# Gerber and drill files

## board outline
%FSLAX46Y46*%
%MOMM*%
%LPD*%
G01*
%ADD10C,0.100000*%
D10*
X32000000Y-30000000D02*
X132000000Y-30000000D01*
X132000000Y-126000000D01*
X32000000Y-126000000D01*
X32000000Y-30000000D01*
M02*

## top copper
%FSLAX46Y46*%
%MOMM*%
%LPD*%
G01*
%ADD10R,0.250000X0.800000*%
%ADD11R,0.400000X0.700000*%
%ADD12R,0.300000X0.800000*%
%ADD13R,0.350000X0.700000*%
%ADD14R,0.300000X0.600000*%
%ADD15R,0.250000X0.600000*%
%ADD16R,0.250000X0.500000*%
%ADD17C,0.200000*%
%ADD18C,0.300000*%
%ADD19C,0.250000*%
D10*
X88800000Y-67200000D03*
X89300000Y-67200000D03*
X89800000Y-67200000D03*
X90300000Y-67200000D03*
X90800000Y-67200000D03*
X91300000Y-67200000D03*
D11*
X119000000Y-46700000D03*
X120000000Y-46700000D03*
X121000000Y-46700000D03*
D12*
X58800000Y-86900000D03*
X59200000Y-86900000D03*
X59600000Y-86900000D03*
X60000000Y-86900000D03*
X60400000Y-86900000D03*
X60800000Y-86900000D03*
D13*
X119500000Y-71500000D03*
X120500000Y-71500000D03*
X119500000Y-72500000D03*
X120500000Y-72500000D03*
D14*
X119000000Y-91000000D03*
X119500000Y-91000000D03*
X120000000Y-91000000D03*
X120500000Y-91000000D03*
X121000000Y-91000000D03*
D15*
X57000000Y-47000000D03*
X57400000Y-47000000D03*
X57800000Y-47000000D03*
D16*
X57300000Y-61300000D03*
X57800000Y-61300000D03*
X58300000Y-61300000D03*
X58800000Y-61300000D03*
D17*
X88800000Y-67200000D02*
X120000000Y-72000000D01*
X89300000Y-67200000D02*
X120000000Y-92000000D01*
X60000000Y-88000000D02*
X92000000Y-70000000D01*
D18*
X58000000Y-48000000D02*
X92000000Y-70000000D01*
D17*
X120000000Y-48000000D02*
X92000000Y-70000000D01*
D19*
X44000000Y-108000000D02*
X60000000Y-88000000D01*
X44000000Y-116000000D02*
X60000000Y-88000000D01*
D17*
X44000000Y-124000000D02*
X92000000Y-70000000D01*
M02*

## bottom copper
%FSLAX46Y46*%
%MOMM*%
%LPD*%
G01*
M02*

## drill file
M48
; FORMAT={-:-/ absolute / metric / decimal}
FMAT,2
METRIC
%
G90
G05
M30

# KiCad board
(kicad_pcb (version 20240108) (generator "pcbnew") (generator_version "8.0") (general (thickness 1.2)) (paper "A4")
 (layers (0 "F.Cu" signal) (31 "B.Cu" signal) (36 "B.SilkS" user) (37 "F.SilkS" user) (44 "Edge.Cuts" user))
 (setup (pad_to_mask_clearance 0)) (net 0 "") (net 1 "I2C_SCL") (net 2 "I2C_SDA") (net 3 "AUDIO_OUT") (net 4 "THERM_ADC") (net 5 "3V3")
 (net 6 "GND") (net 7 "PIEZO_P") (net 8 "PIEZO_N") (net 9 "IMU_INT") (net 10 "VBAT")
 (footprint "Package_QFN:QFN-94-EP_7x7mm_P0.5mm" (layer "F.Cu") (at 92 70)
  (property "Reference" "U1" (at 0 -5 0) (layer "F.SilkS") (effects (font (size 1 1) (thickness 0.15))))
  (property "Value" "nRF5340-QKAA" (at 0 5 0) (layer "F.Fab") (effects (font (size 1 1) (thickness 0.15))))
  (pad "1" smd rect (at -3.2 -2.8) (size 0.25 0.8) (layers "F.Cu" "F.Paste" "F.Mask") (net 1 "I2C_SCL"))
  (pad "2" smd rect (at -2.7 -2.8) (size 0.25 0.8) (layers "F.Cu" "F.Paste" "F.Mask") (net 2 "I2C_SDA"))
  (pad "3" smd rect (at -2.2 -2.8) (size 0.25 0.8) (layers "F.Cu" "F.Paste" "F.Mask") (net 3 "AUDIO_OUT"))
  (pad "4" smd rect (at -1.7 -2.8) (size 0.25 0.8) (layers "F.Cu" "F.Paste" "F.Mask") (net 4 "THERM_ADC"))
  (pad "5" smd rect (at -1.2 -2.8) (size 0.25 0.8) (layers "F.Cu" "F.Paste" "F.Mask") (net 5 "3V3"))
  (pad "6" smd rect (at -0.7 -2.8) (size 0.25 0.8) (layers "F.Cu" "F.Paste" "F.Mask") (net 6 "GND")))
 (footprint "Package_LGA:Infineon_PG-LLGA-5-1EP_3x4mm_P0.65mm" (layer "F.Cu") (at 120 48)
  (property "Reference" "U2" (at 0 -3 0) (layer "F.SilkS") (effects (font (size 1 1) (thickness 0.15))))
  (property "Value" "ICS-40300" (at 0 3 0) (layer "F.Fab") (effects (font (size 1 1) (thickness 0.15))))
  (pad "1" smd rect (at -1.0 -1.3) (size 0.4 0.7) (layers "F.Cu" "F.Paste" "F.Mask") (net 3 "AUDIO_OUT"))
  (pad "2" smd rect (at 0.0 -1.3) (size 0.4 0.7) (layers "F.Cu" "F.Paste" "F.Mask") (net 5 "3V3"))
  (pad "3" smd rect (at 1.0 -1.3) (size 0.4 0.7) (layers "F.Cu" "F.Paste" "F.Mask") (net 6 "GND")))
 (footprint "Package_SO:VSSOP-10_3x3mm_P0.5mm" (layer "F.Cu") (at 60 88)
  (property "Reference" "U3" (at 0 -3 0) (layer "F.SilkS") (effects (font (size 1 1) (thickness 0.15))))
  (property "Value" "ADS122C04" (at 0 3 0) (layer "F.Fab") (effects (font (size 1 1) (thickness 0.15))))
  (pad "1" smd rect (at -1.2 -1.1) (size 0.3 0.8) (layers "F.Cu" "F.Paste" "F.Mask") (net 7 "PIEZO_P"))
  (pad "2" smd rect (at -0.8 -1.1) (size 0.3 0.8) (layers "F.Cu" "F.Paste" "F.Mask") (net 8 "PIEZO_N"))
  (pad "3" smd rect (at -0.4 -1.1) (size 0.3 0.8) (layers "F.Cu" "F.Paste" "F.Mask") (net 1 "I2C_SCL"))
  (pad "4" smd rect (at 0.0 -1.1) (size 0.3 0.8) (layers "F.Cu" "F.Paste" "F.Mask") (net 2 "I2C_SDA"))
  (pad "5" smd rect (at 0.4 -1.1) (size 0.3 0.8) (layers "F.Cu" "F.Paste" "F.Mask") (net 5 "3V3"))
  (pad "6" smd rect (at 0.8 -1.1) (size 0.3 0.8) (layers "F.Cu" "F.Paste" "F.Mask") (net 6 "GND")))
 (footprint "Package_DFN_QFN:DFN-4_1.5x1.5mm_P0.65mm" (layer "F.Cu") (at 120 72)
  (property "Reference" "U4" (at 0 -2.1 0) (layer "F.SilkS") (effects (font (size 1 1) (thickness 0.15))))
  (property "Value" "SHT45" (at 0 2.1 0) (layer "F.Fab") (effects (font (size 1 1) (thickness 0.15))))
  (pad "1" smd rect (at -0.5 -0.5) (size 0.35 0.7) (layers "F.Cu" "F.Paste" "F.Mask") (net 1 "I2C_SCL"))
  (pad "2" smd rect (at 0.5 -0.5) (size 0.35 0.7) (layers "F.Cu" "F.Paste" "F.Mask") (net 2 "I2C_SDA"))
  (pad "3" smd rect (at -0.5 0.5) (size 0.35 0.7) (layers "F.Cu" "F.Paste" "F.Mask") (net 5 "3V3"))
  (pad "4" smd rect (at 0.5 0.5) (size 0.35 0.7) (layers "F.Cu" "F.Paste" "F.Mask") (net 6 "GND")))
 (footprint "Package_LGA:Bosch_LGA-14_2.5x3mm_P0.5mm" (layer "F.Cu") (at 120 92)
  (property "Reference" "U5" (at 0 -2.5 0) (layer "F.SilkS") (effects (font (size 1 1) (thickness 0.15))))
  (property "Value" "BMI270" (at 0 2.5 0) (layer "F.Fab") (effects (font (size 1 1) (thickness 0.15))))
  (pad "1" smd rect (at -1.0 -1.0) (size 0.3 0.6) (layers "F.Cu" "F.Paste" "F.Mask") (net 1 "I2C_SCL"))
  (pad "2" smd rect (at -0.5 -1.0) (size 0.3 0.6) (layers "F.Cu" "F.Paste" "F.Mask") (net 2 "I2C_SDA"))
  (pad "3" smd rect (at 0.0 -1.0) (size 0.3 0.6) (layers "F.Cu" "F.Paste" "F.Mask") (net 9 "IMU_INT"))
  (pad "4" smd rect (at 0.5 -1.0) (size 0.3 0.6) (layers "F.Cu" "F.Paste" "F.Mask") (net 5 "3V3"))
  (pad "5" smd rect (at 1.0 -1.0) (size 0.3 0.6) (layers "F.Cu" "F.Paste" "F.Mask") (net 6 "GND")))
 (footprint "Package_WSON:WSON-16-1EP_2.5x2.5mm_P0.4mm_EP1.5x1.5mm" (layer "F.Cu") (at 58 48)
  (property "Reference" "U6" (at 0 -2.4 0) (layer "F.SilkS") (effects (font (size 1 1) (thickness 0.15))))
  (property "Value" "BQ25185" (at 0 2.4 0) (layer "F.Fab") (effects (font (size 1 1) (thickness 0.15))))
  (pad "1" smd rect (at -1.0 -1.0) (size 0.25 0.6) (layers "F.Cu" "F.Paste" "F.Mask") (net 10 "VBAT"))
  (pad "2" smd rect (at -0.6 -1.0) (size 0.25 0.6) (layers "F.Cu" "F.Paste" "F.Mask") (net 5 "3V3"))
  (pad "3" smd rect (at -0.2 -1.0) (size 0.25 0.6) (layers "F.Cu" "F.Paste" "F.Mask") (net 6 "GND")))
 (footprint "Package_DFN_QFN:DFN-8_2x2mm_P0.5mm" (layer "F.Cu") (at 58 62)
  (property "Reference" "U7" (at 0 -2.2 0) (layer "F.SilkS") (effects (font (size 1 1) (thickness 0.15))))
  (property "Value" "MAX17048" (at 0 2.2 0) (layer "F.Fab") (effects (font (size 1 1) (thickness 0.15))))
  (pad "1" smd rect (at -0.7 -0.7) (size 0.25 0.5) (layers "F.Cu" "F.Paste" "F.Mask") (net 10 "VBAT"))
  (pad "2" smd rect (at -0.2 -0.7) (size 0.25 0.5) (layers "F.Cu" "F.Paste" "F.Mask") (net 1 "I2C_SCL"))
  (pad "3" smd rect (at 0.3 -0.7) (size 0.25 0.5) (layers "F.Cu" "F.Paste" "F.Mask") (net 2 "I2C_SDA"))
  (pad "4" smd rect (at 0.8 -0.7) (size 0.25 0.5) (layers "F.Cu" "F.Paste" "F.Mask") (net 6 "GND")))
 (segment (start 88.8 67.2) (end 120 72) (width 0.2) (layer "F.Cu") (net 1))
 (segment (start 89.3 67.2) (end 120 92) (width 0.2) (layer "F.Cu") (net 2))
 (segment (start 60 88) (end 92 70) (width 0.2) (layer "F.Cu") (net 1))
 (segment (start 58 48) (end 92 70) (width 0.3) (layer "F.Cu") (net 10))
 (segment (start 120 48) (end 92 70) (width 0.2) (layer "F.Cu") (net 3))
 (segment (start 44 108) (end 60 88) (width 0.25) (layer "F.Cu") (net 7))
 (segment (start 44 116) (end 60 88) (width 0.25) (layer "F.Cu") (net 8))
 (segment (start 44 124) (end 92 70) (width 0.2) (layer "F.Cu") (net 4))
 (gr_rect (start 32 30) (end 132 126) (stroke (width 0.1) (type solid)) (fill no) (layer "Edge.Cuts")))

